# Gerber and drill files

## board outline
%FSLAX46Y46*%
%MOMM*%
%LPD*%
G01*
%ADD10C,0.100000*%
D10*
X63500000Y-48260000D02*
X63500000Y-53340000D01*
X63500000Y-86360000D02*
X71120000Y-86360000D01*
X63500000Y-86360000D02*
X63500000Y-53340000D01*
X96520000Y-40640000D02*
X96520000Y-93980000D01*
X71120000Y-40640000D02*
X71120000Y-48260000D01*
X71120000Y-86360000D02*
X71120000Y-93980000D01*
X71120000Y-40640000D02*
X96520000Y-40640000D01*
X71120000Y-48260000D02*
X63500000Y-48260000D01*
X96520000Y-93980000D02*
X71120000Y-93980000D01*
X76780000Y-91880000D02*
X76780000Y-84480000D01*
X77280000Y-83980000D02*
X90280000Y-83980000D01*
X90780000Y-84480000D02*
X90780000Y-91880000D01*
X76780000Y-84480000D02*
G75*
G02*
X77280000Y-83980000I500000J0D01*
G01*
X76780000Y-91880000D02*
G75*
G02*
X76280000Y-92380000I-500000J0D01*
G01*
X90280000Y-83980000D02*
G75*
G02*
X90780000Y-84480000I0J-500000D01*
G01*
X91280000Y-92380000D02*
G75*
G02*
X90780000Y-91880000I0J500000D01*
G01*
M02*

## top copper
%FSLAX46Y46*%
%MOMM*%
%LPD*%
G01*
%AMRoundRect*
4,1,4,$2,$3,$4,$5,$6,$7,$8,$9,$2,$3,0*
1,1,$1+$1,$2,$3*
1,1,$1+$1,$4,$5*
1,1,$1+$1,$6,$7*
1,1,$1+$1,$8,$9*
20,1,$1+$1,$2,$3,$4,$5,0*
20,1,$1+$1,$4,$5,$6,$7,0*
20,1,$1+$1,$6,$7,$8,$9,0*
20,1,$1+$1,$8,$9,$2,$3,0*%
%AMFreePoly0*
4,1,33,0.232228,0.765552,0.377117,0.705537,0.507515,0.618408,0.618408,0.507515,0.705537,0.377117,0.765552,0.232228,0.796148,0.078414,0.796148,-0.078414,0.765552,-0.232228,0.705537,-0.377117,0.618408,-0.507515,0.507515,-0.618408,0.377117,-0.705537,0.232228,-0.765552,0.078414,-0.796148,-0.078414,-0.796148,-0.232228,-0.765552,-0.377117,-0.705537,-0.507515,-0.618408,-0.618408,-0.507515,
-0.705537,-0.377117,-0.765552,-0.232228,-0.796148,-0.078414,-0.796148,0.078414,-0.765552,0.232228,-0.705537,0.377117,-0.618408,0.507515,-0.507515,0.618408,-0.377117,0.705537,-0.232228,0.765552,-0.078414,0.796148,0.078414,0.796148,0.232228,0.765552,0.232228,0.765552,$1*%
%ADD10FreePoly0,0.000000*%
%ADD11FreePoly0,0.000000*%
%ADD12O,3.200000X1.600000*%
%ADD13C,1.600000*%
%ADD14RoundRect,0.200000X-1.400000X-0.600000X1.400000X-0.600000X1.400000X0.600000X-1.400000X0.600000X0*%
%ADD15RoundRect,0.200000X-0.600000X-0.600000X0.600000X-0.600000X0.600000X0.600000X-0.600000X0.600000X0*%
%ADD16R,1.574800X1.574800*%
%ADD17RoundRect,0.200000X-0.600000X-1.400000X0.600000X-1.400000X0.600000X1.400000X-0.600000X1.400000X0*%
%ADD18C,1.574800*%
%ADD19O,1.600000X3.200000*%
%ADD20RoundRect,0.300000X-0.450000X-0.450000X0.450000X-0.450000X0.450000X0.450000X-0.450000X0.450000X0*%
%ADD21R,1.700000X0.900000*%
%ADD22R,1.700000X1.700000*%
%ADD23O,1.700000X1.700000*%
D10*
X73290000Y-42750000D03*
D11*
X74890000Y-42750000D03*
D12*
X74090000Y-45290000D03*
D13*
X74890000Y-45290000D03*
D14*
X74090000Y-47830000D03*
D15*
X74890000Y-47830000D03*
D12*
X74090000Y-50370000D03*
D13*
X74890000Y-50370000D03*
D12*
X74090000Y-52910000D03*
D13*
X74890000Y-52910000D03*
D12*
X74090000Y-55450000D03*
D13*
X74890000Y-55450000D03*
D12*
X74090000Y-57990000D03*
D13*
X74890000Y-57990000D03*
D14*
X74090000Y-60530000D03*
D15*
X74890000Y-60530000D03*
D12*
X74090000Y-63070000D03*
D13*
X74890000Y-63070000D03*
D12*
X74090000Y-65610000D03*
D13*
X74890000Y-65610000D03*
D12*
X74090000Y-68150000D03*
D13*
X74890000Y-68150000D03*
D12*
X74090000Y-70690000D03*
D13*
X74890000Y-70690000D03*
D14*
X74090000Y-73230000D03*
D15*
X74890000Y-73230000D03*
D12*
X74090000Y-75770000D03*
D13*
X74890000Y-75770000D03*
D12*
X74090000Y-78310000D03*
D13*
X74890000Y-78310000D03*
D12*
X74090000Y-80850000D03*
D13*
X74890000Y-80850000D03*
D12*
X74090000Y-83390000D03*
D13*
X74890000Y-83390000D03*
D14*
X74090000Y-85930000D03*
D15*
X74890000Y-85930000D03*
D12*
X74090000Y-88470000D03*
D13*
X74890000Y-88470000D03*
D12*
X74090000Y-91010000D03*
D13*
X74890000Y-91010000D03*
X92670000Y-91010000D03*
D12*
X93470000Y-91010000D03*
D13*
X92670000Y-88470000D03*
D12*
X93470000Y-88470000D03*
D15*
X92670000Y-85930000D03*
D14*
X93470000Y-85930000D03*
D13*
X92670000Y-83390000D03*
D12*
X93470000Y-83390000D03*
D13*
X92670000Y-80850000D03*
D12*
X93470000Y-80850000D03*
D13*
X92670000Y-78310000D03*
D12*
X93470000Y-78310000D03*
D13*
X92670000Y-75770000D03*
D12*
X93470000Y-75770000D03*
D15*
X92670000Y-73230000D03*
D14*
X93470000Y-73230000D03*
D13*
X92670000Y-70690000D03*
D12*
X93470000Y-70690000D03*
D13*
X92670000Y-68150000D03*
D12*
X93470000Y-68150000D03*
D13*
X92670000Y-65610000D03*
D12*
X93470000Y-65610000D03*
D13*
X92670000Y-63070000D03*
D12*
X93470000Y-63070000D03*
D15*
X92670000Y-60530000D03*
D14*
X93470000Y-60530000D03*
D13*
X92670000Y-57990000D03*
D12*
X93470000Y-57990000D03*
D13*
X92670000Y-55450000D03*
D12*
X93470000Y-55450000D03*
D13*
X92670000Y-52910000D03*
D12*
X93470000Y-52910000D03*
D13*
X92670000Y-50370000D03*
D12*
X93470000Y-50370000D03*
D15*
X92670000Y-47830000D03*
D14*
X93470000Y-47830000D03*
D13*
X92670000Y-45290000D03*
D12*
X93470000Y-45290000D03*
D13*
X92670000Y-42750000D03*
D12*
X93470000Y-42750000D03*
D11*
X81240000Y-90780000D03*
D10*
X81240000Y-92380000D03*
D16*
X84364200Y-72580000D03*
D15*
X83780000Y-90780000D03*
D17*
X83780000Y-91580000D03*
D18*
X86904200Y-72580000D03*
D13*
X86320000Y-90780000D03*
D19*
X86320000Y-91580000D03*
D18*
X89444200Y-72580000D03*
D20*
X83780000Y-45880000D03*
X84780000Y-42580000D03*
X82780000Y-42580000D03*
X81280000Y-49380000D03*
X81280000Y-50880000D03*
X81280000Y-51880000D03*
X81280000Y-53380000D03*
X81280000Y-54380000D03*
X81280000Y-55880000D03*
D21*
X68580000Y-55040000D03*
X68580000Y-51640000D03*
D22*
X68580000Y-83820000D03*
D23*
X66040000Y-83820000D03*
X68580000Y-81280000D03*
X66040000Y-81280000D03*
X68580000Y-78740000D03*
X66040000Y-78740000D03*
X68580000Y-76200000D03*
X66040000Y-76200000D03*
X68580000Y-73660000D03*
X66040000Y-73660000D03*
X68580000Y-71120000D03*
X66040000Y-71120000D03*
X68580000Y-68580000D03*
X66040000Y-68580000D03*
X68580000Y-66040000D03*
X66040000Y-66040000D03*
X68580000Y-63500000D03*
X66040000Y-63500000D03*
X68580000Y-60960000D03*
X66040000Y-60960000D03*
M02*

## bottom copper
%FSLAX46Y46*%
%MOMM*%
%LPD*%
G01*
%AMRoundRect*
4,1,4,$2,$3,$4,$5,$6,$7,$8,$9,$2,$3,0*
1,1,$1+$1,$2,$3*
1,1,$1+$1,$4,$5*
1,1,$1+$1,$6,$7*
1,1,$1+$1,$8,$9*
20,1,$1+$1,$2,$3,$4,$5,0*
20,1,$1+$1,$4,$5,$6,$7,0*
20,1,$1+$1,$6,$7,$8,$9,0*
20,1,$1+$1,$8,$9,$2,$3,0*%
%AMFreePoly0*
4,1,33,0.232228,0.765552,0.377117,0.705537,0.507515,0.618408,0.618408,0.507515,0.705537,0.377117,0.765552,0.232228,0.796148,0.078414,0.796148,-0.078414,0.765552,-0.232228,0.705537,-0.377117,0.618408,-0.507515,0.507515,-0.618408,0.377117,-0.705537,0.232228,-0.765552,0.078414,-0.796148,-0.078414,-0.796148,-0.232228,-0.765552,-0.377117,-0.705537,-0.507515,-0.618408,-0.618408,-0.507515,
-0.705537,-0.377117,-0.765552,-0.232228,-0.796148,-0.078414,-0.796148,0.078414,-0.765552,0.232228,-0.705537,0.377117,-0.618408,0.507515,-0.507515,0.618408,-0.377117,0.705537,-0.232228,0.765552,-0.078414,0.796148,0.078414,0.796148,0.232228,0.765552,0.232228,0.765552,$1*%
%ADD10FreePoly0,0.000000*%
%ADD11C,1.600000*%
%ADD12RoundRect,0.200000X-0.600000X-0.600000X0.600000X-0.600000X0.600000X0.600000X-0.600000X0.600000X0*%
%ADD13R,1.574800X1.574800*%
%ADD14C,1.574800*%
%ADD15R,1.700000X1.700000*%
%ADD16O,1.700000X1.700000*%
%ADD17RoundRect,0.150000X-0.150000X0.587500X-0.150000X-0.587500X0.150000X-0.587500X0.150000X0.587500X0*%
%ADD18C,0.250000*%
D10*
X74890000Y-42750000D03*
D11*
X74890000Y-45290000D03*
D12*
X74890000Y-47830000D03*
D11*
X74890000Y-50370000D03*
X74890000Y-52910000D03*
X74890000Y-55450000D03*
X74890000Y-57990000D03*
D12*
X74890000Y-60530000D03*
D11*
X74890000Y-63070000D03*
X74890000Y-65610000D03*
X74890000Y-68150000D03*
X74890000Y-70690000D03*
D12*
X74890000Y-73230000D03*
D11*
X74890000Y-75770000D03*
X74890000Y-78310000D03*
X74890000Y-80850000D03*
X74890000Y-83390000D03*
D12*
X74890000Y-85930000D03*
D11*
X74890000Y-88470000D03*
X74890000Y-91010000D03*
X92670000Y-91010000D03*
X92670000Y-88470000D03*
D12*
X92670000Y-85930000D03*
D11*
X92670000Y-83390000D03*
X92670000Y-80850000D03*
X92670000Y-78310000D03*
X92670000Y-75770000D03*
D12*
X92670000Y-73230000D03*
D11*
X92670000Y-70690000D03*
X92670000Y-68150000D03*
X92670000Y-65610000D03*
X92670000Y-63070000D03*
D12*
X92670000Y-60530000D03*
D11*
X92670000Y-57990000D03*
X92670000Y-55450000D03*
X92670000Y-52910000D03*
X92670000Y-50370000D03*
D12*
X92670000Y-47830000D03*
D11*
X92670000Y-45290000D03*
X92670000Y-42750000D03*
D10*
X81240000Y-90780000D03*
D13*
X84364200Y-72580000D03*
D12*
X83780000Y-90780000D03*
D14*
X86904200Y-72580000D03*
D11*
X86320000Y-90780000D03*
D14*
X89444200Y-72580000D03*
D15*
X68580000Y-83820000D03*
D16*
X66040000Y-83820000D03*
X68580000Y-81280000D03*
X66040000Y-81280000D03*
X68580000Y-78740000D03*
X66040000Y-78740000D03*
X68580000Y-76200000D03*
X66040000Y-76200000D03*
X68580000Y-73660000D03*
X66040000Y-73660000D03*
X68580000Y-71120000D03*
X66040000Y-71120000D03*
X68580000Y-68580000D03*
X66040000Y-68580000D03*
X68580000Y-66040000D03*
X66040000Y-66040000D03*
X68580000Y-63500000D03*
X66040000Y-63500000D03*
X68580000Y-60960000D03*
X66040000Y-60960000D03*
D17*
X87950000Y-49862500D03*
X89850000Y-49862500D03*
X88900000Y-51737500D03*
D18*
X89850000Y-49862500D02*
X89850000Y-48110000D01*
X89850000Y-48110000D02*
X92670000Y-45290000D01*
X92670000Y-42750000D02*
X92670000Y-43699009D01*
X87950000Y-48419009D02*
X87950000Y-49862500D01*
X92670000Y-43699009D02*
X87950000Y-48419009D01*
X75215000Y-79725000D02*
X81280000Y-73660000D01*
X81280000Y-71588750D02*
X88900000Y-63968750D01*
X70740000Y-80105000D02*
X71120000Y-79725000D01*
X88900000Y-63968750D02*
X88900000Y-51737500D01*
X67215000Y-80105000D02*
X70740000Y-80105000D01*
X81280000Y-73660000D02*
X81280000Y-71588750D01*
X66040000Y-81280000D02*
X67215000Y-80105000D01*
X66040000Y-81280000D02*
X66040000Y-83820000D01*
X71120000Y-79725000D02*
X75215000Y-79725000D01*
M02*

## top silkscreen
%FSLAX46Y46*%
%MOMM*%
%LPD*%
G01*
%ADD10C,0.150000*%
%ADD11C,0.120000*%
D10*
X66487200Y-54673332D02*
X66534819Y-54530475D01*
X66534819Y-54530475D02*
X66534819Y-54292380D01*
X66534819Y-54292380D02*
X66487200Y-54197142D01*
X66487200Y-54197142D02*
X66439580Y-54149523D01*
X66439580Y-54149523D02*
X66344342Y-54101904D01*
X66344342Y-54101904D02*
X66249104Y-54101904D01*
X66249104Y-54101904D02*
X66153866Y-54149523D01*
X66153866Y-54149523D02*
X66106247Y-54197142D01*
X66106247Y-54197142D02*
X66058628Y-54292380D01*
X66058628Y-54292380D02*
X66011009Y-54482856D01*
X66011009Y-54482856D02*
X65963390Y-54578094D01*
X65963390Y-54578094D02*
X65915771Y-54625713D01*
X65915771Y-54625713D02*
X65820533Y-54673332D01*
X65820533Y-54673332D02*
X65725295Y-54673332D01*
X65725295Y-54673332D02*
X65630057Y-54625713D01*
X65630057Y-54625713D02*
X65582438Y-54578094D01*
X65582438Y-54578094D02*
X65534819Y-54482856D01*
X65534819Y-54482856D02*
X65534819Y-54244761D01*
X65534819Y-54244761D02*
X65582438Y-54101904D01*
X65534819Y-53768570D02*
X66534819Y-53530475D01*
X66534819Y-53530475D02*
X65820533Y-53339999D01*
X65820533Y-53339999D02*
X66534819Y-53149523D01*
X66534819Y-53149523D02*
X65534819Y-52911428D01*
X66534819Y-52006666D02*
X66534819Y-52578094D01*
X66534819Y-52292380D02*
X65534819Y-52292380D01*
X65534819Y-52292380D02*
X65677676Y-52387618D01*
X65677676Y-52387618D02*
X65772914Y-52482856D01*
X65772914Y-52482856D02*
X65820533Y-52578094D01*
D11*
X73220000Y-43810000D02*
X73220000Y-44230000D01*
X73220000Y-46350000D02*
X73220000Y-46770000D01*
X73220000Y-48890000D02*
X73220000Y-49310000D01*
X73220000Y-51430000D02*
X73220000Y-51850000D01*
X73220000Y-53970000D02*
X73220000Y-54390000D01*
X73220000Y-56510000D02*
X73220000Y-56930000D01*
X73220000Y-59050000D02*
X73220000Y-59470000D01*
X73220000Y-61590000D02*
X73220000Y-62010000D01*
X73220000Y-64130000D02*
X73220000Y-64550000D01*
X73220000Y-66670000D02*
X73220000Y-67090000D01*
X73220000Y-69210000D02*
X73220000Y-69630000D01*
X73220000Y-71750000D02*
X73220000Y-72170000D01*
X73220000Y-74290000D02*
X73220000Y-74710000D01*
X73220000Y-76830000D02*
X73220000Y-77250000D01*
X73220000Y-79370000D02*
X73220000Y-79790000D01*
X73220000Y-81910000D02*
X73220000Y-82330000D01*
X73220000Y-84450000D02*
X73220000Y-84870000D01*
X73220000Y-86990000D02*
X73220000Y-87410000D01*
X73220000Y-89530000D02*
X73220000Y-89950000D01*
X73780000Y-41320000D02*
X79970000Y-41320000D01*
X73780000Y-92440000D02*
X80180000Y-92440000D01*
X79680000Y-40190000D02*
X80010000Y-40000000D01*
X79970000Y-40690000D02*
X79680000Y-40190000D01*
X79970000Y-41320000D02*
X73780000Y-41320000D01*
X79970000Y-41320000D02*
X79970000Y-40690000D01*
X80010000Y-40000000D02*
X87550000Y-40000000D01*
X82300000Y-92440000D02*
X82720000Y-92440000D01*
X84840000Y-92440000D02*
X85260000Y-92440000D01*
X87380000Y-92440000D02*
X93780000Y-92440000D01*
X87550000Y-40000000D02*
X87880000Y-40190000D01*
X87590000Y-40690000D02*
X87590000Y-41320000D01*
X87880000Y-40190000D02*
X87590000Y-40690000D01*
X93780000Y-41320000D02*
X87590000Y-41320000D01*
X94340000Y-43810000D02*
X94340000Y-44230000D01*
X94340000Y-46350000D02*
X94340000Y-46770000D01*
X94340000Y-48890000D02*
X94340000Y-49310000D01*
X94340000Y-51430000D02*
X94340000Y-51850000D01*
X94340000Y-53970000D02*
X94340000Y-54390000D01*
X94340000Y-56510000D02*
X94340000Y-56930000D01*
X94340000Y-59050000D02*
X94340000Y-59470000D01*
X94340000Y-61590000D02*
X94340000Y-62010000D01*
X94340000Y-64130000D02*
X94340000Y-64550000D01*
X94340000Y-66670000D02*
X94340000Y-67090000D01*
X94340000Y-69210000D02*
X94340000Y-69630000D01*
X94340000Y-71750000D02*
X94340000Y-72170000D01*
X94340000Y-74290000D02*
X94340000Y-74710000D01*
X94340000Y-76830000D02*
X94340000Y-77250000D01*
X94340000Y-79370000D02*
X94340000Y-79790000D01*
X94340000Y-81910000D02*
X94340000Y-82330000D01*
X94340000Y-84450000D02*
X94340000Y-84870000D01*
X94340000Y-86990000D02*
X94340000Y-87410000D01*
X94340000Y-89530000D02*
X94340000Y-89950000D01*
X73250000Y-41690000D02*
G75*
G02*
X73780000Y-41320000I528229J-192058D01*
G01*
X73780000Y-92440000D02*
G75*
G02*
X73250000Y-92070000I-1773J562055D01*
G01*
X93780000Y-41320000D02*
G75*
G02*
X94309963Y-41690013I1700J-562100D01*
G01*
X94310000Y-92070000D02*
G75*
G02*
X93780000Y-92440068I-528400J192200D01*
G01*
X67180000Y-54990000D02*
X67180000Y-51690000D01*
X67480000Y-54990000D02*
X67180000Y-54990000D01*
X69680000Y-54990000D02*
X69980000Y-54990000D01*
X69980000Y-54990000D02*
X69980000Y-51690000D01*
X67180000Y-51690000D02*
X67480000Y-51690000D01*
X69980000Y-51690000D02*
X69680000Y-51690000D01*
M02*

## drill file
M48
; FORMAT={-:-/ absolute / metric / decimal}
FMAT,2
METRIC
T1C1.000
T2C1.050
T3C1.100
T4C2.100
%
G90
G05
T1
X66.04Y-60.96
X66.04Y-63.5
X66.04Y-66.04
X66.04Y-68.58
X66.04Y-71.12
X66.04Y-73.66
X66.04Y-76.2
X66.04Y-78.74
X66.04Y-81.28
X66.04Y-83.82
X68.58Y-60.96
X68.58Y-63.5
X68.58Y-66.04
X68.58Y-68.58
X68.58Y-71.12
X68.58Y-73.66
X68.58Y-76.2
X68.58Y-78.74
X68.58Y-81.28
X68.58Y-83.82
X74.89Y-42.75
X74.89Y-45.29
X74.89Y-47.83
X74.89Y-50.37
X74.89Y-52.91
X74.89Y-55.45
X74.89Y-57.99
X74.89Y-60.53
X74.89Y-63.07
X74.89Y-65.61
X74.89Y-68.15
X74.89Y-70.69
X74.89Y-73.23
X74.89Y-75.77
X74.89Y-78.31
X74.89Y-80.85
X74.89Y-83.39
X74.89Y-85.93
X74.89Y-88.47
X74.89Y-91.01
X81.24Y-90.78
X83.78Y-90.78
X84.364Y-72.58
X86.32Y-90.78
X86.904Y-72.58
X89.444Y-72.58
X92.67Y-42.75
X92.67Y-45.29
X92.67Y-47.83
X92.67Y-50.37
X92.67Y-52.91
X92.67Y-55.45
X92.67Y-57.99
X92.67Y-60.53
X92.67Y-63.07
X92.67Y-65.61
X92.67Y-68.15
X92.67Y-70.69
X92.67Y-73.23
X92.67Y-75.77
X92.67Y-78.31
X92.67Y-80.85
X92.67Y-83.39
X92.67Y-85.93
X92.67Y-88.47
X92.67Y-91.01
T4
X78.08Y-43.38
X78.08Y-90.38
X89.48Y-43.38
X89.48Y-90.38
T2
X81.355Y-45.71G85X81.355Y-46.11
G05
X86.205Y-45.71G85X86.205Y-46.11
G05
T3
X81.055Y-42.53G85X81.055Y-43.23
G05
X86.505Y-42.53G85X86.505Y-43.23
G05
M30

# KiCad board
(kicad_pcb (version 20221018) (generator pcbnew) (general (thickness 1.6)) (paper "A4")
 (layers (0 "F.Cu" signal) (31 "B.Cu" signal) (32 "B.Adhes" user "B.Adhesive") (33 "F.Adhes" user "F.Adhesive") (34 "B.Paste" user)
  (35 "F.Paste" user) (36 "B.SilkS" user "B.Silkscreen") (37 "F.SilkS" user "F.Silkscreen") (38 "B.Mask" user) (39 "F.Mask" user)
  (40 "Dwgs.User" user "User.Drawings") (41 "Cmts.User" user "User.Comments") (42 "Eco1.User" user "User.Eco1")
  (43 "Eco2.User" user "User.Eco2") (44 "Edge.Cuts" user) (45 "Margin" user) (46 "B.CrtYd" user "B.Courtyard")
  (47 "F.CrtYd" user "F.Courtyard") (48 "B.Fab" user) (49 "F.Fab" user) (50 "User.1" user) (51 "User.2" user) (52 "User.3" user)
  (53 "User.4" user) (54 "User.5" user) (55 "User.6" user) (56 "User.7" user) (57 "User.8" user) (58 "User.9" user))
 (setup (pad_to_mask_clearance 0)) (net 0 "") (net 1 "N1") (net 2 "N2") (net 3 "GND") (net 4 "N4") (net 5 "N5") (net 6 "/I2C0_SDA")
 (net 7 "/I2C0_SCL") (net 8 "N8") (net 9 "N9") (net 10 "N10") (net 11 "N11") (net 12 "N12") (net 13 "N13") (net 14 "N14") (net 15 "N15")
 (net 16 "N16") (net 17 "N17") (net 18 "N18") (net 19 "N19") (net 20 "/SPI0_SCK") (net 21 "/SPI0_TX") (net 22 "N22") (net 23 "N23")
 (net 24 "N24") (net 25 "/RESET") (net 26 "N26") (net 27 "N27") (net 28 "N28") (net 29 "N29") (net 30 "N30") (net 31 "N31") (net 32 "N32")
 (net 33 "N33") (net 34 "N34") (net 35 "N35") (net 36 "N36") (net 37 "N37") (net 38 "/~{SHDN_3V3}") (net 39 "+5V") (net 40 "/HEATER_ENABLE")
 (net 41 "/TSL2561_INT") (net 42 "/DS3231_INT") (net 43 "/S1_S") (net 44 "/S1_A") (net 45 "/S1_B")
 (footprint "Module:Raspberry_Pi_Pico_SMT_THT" (layer "F.Cu") (at 74.89 42.75)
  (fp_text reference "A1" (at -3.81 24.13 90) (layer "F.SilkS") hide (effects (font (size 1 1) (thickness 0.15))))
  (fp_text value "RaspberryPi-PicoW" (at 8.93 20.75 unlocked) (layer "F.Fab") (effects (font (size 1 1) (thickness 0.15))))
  (fp_line (start -1.67 1.06) (end -1.67 1.48) (stroke (width 0.12) (type solid)) (layer "F.SilkS"))
  (fp_line (start -1.67 3.6) (end -1.67 4.02) (stroke (width 0.12) (type solid)) (layer "F.SilkS"))
  (fp_line (start -1.67 6.14) (end -1.67 6.56) (stroke (width 0.12) (type solid)) (layer "F.SilkS"))
  (fp_line (start -1.67 8.68) (end -1.67 9.1) (stroke (width 0.12) (type solid)) (layer "F.SilkS"))
  (fp_line (start -1.67 11.22) (end -1.67 11.64) (stroke (width 0.12) (type solid)) (layer "F.SilkS"))
  (fp_line (start -1.67 13.76) (end -1.67 14.18) (stroke (width 0.12) (type solid)) (layer "F.SilkS"))
  (fp_line (start -1.67 16.3) (end -1.67 16.72) (stroke (width 0.12) (type solid)) (layer "F.SilkS"))
  (fp_line (start -1.67 18.84) (end -1.67 19.26) (stroke (width 0.12) (type solid)) (layer "F.SilkS"))
  (fp_line (start -1.67 21.38) (end -1.67 21.8) (stroke (width 0.12) (type solid)) (layer "F.SilkS"))
  (fp_line (start -1.67 23.92) (end -1.67 24.34) (stroke (width 0.12) (type solid)) (layer "F.SilkS"))
  (fp_line (start -1.67 26.46) (end -1.67 26.88) (stroke (width 0.12) (type solid)) (layer "F.SilkS"))
  (fp_line (start -1.67 29) (end -1.67 29.42) (stroke (width 0.12) (type solid)) (layer "F.SilkS"))
  (fp_line (start -1.67 31.54) (end -1.67 31.96) (stroke (width 0.12) (type solid)) (layer "F.SilkS"))
  (fp_line (start -1.67 34.08) (end -1.67 34.5) (stroke (width 0.12) (type solid)) (layer "F.SilkS"))
  (fp_line (start -1.67 36.62) (end -1.67 37.04) (stroke (width 0.12) (type solid)) (layer "F.SilkS"))
  (fp_line (start -1.67 39.16) (end -1.67 39.58) (stroke (width 0.12) (type solid)) (layer "F.SilkS"))
  (fp_line (start -1.67 41.7) (end -1.67 42.12) (stroke (width 0.12) (type solid)) (layer "F.SilkS"))
  (fp_line (start -1.67 44.24) (end -1.67 44.66) (stroke (width 0.12) (type solid)) (layer "F.SilkS"))
  (fp_line (start -1.67 46.78) (end -1.67 47.2) (stroke (width 0.12) (type solid)) (layer "F.SilkS"))
  (fp_line (start -1.11 -1.43) (end 5.08 -1.43) (stroke (width 0.12) (type solid)) (layer "F.SilkS"))
  (fp_line (start -1.11 49.69) (end 5.29 49.69) (stroke (width 0.12) (type solid)) (layer "F.SilkS"))
  (fp_line (start 4.79 -2.56) (end 5.12 -2.75) (stroke (width 0.12) (type solid)) (layer "F.SilkS"))
  (fp_line (start 5.08 -2.06) (end 4.79 -2.56) (stroke (width 0.12) (type solid)) (layer "F.SilkS"))
  (fp_line (start 5.08 -1.43) (end -1.11 -1.43) (stroke (width 0.12) (type solid)) (layer "F.SilkS"))
  (fp_line (start 5.08 -1.43) (end 5.08 -2.06) (stroke (width 0.12) (type solid)) (layer "F.SilkS"))
  (fp_line (start 5.12 -2.75) (end 12.66 -2.75) (stroke (width 0.12) (type solid)) (layer "F.SilkS"))
  (fp_line (start 7.41 49.69) (end 7.83 49.69) (stroke (width 0.12) (type solid)) (layer "F.SilkS"))
  (fp_line (start 9.95 49.69) (end 10.37 49.69) (stroke (width 0.12) (type solid)) (layer "F.SilkS"))
  (fp_line (start 12.49 49.69) (end 18.89 49.69) (stroke (width 0.12) (type solid)) (layer "F.SilkS"))
  (fp_line (start 12.66 -2.75) (end 12.99 -2.56) (stroke (width 0.12) (type solid)) (layer "F.SilkS"))
  (fp_line (start 12.7 -2.06) (end 12.7 -1.43) (stroke (width 0.12) (type solid)) (layer "F.SilkS"))
  (fp_line (start 12.99 -2.56) (end 12.7 -2.06) (stroke (width 0.12) (type solid)) (layer "F.SilkS"))
  (fp_line (start 18.89 -1.43) (end 12.7 -1.43) (stroke (width 0.12) (type solid)) (layer "F.SilkS"))
  (fp_line (start 19.45 1.06) (end 19.45 1.48) (stroke (width 0.12) (type solid)) (layer "F.SilkS"))
  (fp_line (start 19.45 3.6) (end 19.45 4.02) (stroke (width 0.12) (type solid)) (layer "F.SilkS"))
  (fp_line (start 19.45 6.14) (end 19.45 6.56) (stroke (width 0.12) (type solid)) (layer "F.SilkS"))
  (fp_line (start 19.45 8.68) (end 19.45 9.1) (stroke (width 0.12) (type solid)) (layer "F.SilkS"))
  (fp_line (start 19.45 11.22) (end 19.45 11.64) (stroke (width 0.12) (type solid)) (layer "F.SilkS"))
  (fp_line (start 19.45 13.76) (end 19.45 14.18) (stroke (width 0.12) (type solid)) (layer "F.SilkS"))
  (fp_line (start 19.45 16.3) (end 19.45 16.72) (stroke (width 0.12) (type solid)) (layer "F.SilkS"))
  (fp_line (start 19.45 18.84) (end 19.45 19.26) (stroke (width 0.12) (type solid)) (layer "F.SilkS"))
  (fp_line (start 19.45 21.38) (end 19.45 21.8) (stroke (width 0.12) (type solid)) (layer "F.SilkS"))
  (fp_line (start 19.45 23.92) (end 19.45 24.34) (stroke (width 0.12) (type solid)) (layer "F.SilkS"))
  (fp_line (start 19.45 26.46) (end 19.45 26.88) (stroke (width 0.12) (type solid)) (layer "F.SilkS"))
  (fp_line (start 19.45 29) (end 19.45 29.42) (stroke (width 0.12) (type solid)) (layer "F.SilkS"))
  (fp_line (start 19.45 31.54) (end 19.45 31.96) (stroke (width 0.12) (type solid)) (layer "F.SilkS"))
  (fp_line (start 19.45 34.08) (end 19.45 34.5) (stroke (width 0.12) (type solid)) (layer "F.SilkS"))
  (fp_line (start 19.45 36.62) (end 19.45 37.04) (stroke (width 0.12) (type solid)) (layer "F.SilkS"))
  (fp_line (start 19.45 39.16) (end 19.45 39.58) (stroke (width 0.12) (type solid)) (layer "F.SilkS"))
  (fp_line (start 19.45 41.7) (end 19.45 42.12) (stroke (width 0.12) (type solid)) (layer "F.SilkS"))
  (fp_line (start 19.45 44.24) (end 19.45 44.66) (stroke (width 0.12) (type solid)) (layer "F.SilkS"))
  (fp_line (start 19.45 46.78) (end 19.45 47.2) (stroke (width 0.12) (type solid)) (layer "F.SilkS"))
  (fp_arc (start -1.64 -1.06) (mid -1.433508 -1.328808) (end -1.11 -1.43) (stroke (width 0.12) (type solid)) (layer "F.SilkS"))
  (fp_arc (start -1.11 49.69) (mid -1.433508 49.588809) (end -1.64 49.32) (stroke (width 0.12) (type solid)) (layer "F.SilkS"))
  (fp_arc (start 18.89 -1.43) (mid 19.213502 -1.328793) (end 19.42 -1.06) (stroke (width 0.12) (type solid)) (layer "F.SilkS"))
  (fp_arc (start 19.42 49.32) (mid 19.213487 49.588772) (end 18.89 49.69) (stroke (width 0.12) (type solid)) (layer "F.SilkS"))
  (fp_line (start 1.89 49.13) (end 1.89 41.73) (stroke (width 0.1) (type solid)) (layer "Edge.Cuts"))
  (fp_line (start 2.39 41.23) (end 15.39 41.23) (stroke (width 0.1) (type solid)) (layer "Edge.Cuts"))
  (fp_line (start 15.89 41.73) (end 15.89 49.13) (stroke (width 0.1) (type solid)) (layer "Edge.Cuts"))
  (fp_arc (start 1.89 41.73) (mid 2.036447 41.376447) (end 2.39 41.23) (stroke (width 0.1) (type solid)) (layer "Edge.Cuts"))
  (fp_arc (start 1.89 49.13) (mid 1.743553 49.483553) (end 1.39 49.63) (stroke (width 0.1) (type solid)) (layer "Edge.Cuts"))
  (fp_arc (start 15.39 41.23) (mid 15.743553 41.376447) (end 15.89 41.73) (stroke (width 0.1) (type solid)) (layer "Edge.Cuts"))
  (fp_arc (start 16.39 49.63) (mid 16.036447 49.483553) (end 15.89 49.13) (stroke (width 0.1) (type solid)) (layer "Edge.Cuts"))
  (pad "" np_thru_hole circle (at 3.19 0.63) (size 2.1 2.1) (drill 2.1) (layers "F&B.Cu" "*.Mask") (solder_mask_margin 0.85)
   (clearance 1.05))
  (pad "" np_thru_hole circle (at 3.19 47.63) (size 2.1 2.1) (drill 2.1) (layers "F&B.Cu" "*.Mask") (solder_mask_margin 0.85)
   (clearance 1.05))
  (pad "" np_thru_hole oval (at 6.165 0.13) (size 1.1 1.8) (drill oval 1.1 1.8) (layers "*.Mask"))
  (pad "" np_thru_hole oval (at 6.465 3.16) (size 1.05 1.45) (drill oval 1.05 1.45) (layers "*.Mask"))
  (pad "" np_thru_hole oval (at 11.315 3.16) (size 1.05 1.45) (drill oval 1.05 1.45) (layers "*.Mask"))
  (pad "" np_thru_hole oval (at 11.615 0.13) (size 1.1 1.8) (drill oval 1.1 1.8) (layers "*.Mask"))
  (pad "" np_thru_hole circle (at 14.59 0.63) (size 2.1 2.1) (drill 2.1) (layers "F&B.Cu" "*.Mask") (solder_mask_margin 0.85)
   (clearance 1.05))
  (pad "" np_thru_hole circle (at 14.59 47.63) (size 2.1 2.1) (drill 2.1) (layers "F&B.Cu" "*.Mask") (solder_mask_margin 0.85)
   (clearance 1.05))
  (pad "1" smd custom (at -1.6 0) (size 1.6 1.6) (layers "F.Cu" "F.Mask") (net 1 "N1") (thermal_bridge_angle 45)
   (options (clearance convexhull) (anchor circle)) (primitives))
  (pad "1" thru_hole custom (at 0 0) (size 1.6 1.6) (drill 1) (layers "*.Cu" "*.Mask") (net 1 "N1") (thermal_bridge_angle 45)
   (options (clearance convexhull) (anchor circle)) (primitives))
  (pad "2" smd oval (at -1.6 2.54) (size 3.2 1.6) (drill (offset 0.8 0)) (layers "F.Cu" "F.Mask") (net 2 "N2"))
  (pad "2" thru_hole circle (at 0 2.54) (size 1.6 1.6) (drill 1) (layers "*.Cu" "*.Mask") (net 2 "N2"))
  (pad "3" smd roundrect (at -1.6 5.08) (size 3.2 1.6) (drill (offset 0.8 0)) (layers "F.Cu" "F.Mask") (roundrect_rratio 0.125)
   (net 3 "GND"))
  (pad "3" thru_hole roundrect (at 0 5.08) (size 1.6 1.6) (drill 1) (layers "*.Cu" "*.Mask") (roundrect_rratio 0.125) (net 3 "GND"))
  (pad "4" smd oval (at -1.6 7.62) (size 3.2 1.6) (drill (offset 0.8 0)) (layers "F.Cu" "F.Mask") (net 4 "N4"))
  (pad "4" thru_hole circle (at 0 7.62) (size 1.6 1.6) (drill 1) (layers "*.Cu" "*.Mask") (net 4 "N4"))
  (pad "5" smd oval (at -1.6 10.16) (size 3.2 1.6) (drill (offset 0.8 0)) (layers "F.Cu" "F.Mask") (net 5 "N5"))
  (pad "5" thru_hole circle (at 0 10.16) (size 1.6 1.6) (drill 1) (layers "*.Cu" "*.Mask") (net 5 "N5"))
  (pad "6" smd oval (at -1.6 12.7) (size 3.2 1.6) (drill (offset 0.8 0)) (layers "F.Cu" "F.Mask") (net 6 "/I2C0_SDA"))
  (pad "6" thru_hole circle (at 0 12.7) (size 1.6 1.6) (drill 1) (layers "*.Cu" "*.Mask") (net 6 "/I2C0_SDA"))
  (pad "7" smd oval (at -1.6 15.24) (size 3.2 1.6) (drill (offset 0.8 0)) (layers "F.Cu" "F.Mask") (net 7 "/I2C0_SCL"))
  (pad "7" thru_hole circle (at 0 15.24) (size 1.6 1.6) (drill 1) (layers "*.Cu" "*.Mask") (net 7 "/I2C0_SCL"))
  (pad "8" smd roundrect (at -1.6 17.78) (size 3.2 1.6) (drill (offset 0.8 0)) (layers "F.Cu" "F.Mask") (roundrect_rratio 0.125)
   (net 3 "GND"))
  (pad "8" thru_hole roundrect (at 0 17.78) (size 1.6 1.6) (drill 1) (layers "*.Cu" "*.Mask") (roundrect_rratio 0.125) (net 3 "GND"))
  (pad "9" smd oval (at -1.6 20.32) (size 3.2 1.6) (drill (offset 0.8 0)) (layers "F.Cu" "F.Mask") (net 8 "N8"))
  (pad "9" thru_hole circle (at 0 20.32) (size 1.6 1.6) (drill 1) (layers "*.Cu" "*.Mask") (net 8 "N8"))
  (pad "10" smd oval (at -1.6 22.86) (size 3.2 1.6) (drill (offset 0.8 0)) (layers "F.Cu" "F.Mask") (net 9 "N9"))
  (pad "10" thru_hole circle (at 0 22.86) (size 1.6 1.6) (drill 1) (layers "*.Cu" "*.Mask") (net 9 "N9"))
  (pad "11" smd oval (at -1.6 25.4) (size 3.2 1.6) (drill (offset 0.8 0)) (layers "F.Cu" "F.Mask") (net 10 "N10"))
  (pad "11" thru_hole circle (at 0 25.4) (size 1.6 1.6) (drill 1) (layers "*.Cu" "*.Mask") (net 10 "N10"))
  (pad "12" smd oval (at -1.6 27.94) (size 3.2 1.6) (drill (offset 0.8 0)) (layers "F.Cu" "F.Mask") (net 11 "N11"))
  (pad "12" thru_hole circle (at 0 27.94) (size 1.6 1.6) (drill 1) (layers "*.Cu" "*.Mask") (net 11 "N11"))
  (pad "13" smd roundrect (at -1.6 30.48) (size 3.2 1.6) (drill (offset 0.8 0)) (layers "F.Cu" "F.Mask") (roundrect_rratio 0.125)
   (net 3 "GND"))
  (pad "13" thru_hole roundrect (at 0 30.48) (size 1.6 1.6) (drill 1) (layers "*.Cu" "*.Mask") (roundrect_rratio 0.125) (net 3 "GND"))
  (pad "14" smd oval (at -1.6 33.02) (size 3.2 1.6) (drill (offset 0.8 0)) (layers "F.Cu" "F.Mask") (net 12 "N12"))
  (pad "14" thru_hole circle (at 0 33.02) (size 1.6 1.6) (drill 1) (layers "*.Cu" "*.Mask") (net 12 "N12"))
  (pad "15" smd oval (at -1.6 35.56) (size 3.2 1.6) (drill (offset 0.8 0)) (layers "F.Cu" "F.Mask") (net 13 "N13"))
  (pad "15" thru_hole circle (at 0 35.56) (size 1.6 1.6) (drill 1) (layers "*.Cu" "*.Mask") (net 13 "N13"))
  (pad "16" smd oval (at -1.6 38.1) (size 3.2 1.6) (drill (offset 0.8 0)) (layers "F.Cu" "F.Mask") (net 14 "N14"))
  (pad "16" thru_hole circle (at 0 38.1) (size 1.6 1.6) (drill 1) (layers "*.Cu" "*.Mask") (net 14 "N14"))
  (pad "17" smd oval (at -1.6 40.64) (size 3.2 1.6) (drill (offset 0.8 0)) (layers "F.Cu" "F.Mask") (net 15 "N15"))
  (pad "17" thru_hole circle (at 0 40.64) (size 1.6 1.6) (drill 1) (layers "*.Cu" "*.Mask") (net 15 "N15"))
  (pad "18" smd roundrect (at -1.6 43.18) (size 3.2 1.6) (drill (offset 0.8 0)) (layers "F.Cu" "F.Mask") (roundrect_rratio 0.125)
   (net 3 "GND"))
  (pad "18" thru_hole roundrect (at 0 43.18) (size 1.6 1.6) (drill 1) (layers "*.Cu" "*.Mask") (roundrect_rratio 0.125) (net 3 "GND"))
  (pad "19" smd oval (at -1.6 45.72) (size 3.2 1.6) (drill (offset 0.8 0)) (layers "F.Cu" "F.Mask") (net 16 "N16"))
  (pad "19" thru_hole circle (at 0 45.72) (size 1.6 1.6) (drill 1) (layers "*.Cu" "*.Mask") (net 16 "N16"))
  (pad "20" smd oval (at -1.6 48.26) (size 3.2 1.6) (drill (offset 0.8 0)) (layers "F.Cu" "F.Mask") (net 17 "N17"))
  (pad "20" thru_hole circle (at 0 48.26) (size 1.6 1.6) (drill 1) (layers "*.Cu" "*.Mask") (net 17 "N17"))
  (pad "21" thru_hole circle (at 17.78 48.26) (size 1.6 1.6) (drill 1) (layers "*.Cu" "*.Mask") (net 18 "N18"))
  (pad "21" smd oval (at 19.38 48.26) (size 3.2 1.6) (drill (offset -0.8 0)) (layers "F.Cu" "F.Mask") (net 18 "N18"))
  (pad "22" thru_hole circle (at 17.78 45.72) (size 1.6 1.6) (drill 1) (layers "*.Cu" "*.Mask") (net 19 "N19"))
  (pad "22" smd oval (at 19.38 45.72) (size 3.2 1.6) (drill (offset -0.8 0)) (layers "F.Cu" "F.Mask") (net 19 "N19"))
  (pad "23" thru_hole roundrect (at 17.78 43.18) (size 1.6 1.6) (drill 1) (layers "*.Cu" "*.Mask") (roundrect_rratio 0.125) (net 3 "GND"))
  (pad "23" smd roundrect (at 19.38 43.18) (size 3.2 1.6) (drill (offset -0.8 0)) (layers "F.Cu" "F.Mask") (roundrect_rratio 0.125)
   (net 3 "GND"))
  (pad "24" thru_hole circle (at 17.78 40.64) (size 1.6 1.6) (drill 1) (layers "*.Cu" "*.Mask") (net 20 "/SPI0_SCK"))
  (pad "24" smd oval (at 19.38 40.64) (size 3.2 1.6) (drill (offset -0.8 0)) (layers "F.Cu" "F.Mask") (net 20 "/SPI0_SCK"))
  (pad "25" thru_hole circle (at 17.78 38.1) (size 1.6 1.6) (drill 1) (layers "*.Cu" "*.Mask") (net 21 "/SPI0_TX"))
  (pad "25" smd oval (at 19.38 38.1) (size 3.2 1.6) (drill (offset -0.8 0)) (layers "F.Cu" "F.Mask") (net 21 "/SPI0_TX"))
  (pad "26" thru_hole circle (at 17.78 35.56) (size 1.6 1.6) (drill 1) (layers "*.Cu" "*.Mask") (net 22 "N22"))
  (pad "26" smd oval (at 19.38 35.56) (size 3.2 1.6) (drill (offset -0.8 0)) (layers "F.Cu" "F.Mask") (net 22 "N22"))
  (pad "27" thru_hole circle (at 17.78 33.02) (size 1.6 1.6) (drill 1) (layers "*.Cu" "*.Mask") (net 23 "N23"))
  (pad "27" smd oval (at 19.38 33.02) (size 3.2 1.6) (drill (offset -0.8 0)) (layers "F.Cu" "F.Mask") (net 23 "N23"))
  (pad "28" thru_hole roundrect (at 17.78 30.48) (size 1.6 1.6) (drill 1) (layers "*.Cu" "*.Mask") (roundrect_rratio 0.125) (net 3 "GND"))
  (pad "28" smd roundrect (at 19.38 30.48) (size 3.2 1.6) (drill (offset -0.8 0)) (layers "F.Cu" "F.Mask") (roundrect_rratio 0.125)
   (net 3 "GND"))
  (pad "29" thru_hole circle (at 17.78 27.94) (size 1.6 1.6) (drill 1) (layers "*.Cu" "*.Mask") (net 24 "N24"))
  (pad "29" smd oval (at 19.38 27.94) (size 3.2 1.6) (drill (offset -0.8 0)) (layers "F.Cu" "F.Mask") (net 24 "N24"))
  (pad "30" thru_hole circle (at 17.78 25.4) (size 1.6 1.6) (drill 1) (layers "*.Cu" "*.Mask") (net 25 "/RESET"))
  (pad "30" smd oval (at 19.38 25.4) (size 3.2 1.6) (drill (offset -0.8 0)) (layers "F.Cu" "F.Mask") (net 25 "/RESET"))
  (pad "31" thru_hole circle (at 17.78 22.86) (size 1.6 1.6) (drill 1) (layers "*.Cu" "*.Mask") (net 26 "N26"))
  (pad "31" smd oval (at 19.38 22.86) (size 3.2 1.6) (drill (offset -0.8 0)) (layers "F.Cu" "F.Mask") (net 26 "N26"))
  (pad "32" thru_hole circle (at 17.78 20.32) (size 1.6 1.6) (drill 1) (layers "*.Cu" "*.Mask") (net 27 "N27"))
  (pad "32" smd oval (at 19.38 20.32) (size 3.2 1.6) (drill (offset -0.8 0)) (layers "F.Cu" "F.Mask") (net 27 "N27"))
  (pad "33" thru_hole roundrect (at 17.78 17.78) (size 1.6 1.6) (drill 1) (layers "*.Cu" "*.Mask") (roundrect_rratio 0.125) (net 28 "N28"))
  (pad "33" smd roundrect (at 19.38 17.78) (size 3.2 1.6) (drill (offset -0.8 0)) (layers "F.Cu" "F.Mask") (roundrect_rratio 0.125)
   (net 28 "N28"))
  (pad "34" thru_hole circle (at 17.78 15.24) (size 1.6 1.6) (drill 1) (layers "*.Cu" "*.Mask") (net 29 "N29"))
  (pad "34" smd oval (at 19.38 15.24) (size 3.2 1.6) (drill (offset -0.8 0)) (layers "F.Cu" "F.Mask") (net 29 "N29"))
  (pad "35" thru_hole circle (at 17.78 12.7) (size 1.6 1.6) (drill 1) (layers "*.Cu" "*.Mask") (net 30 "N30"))
  (pad "35" smd oval (at 19.38 12.7) (size 3.2 1.6) (drill (offset -0.8 0)) (layers "F.Cu" "F.Mask") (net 30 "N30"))
  (pad "36" thru_hole circle (at 17.78 10.16) (size 1.6 1.6) (drill 1) (layers "*.Cu" "*.Mask") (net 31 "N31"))
  (pad "36" smd oval (at 19.38 10.16) (size 3.2 1.6) (drill (offset -0.8 0)) (layers "F.Cu" "F.Mask") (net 31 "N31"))
  (pad "37" thru_hole circle (at 17.78 7.62) (size 1.6 1.6) (drill 1) (layers "*.Cu" "*.Mask") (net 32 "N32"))
  (pad "37" smd oval (at 19.38 7.62) (size 3.2 1.6) (drill (offset -0.8 0)) (layers "F.Cu" "F.Mask") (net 32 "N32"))
  (pad "38" thru_hole roundrect (at 17.78 5.08) (size 1.6 1.6) (drill 1) (layers "*.Cu" "*.Mask") (roundrect_rratio 0.125) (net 3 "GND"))
  (pad "38" smd roundrect (at 19.38 5.08) (size 3.2 1.6) (drill (offset -0.8 0)) (layers "F.Cu" "F.Mask") (roundrect_rratio 0.125)
   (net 3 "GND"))
  (pad "39" thru_hole circle (at 17.78 2.54) (size 1.6 1.6) (drill 1) (layers "*.Cu" "*.Mask") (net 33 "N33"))
  (pad "39" smd oval (at 19.38 2.54) (size 3.2 1.6) (drill (offset -0.8 0)) (layers "F.Cu" "F.Mask") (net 33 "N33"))
  (pad "40" thru_hole circle (at 17.78 0) (size 1.6 1.6) (drill 1) (layers "*.Cu" "*.Mask") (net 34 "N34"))
  (pad "40" smd oval (at 19.38 0) (size 3.2 1.6) (drill (offset -0.8 0)) (layers "F.Cu" "F.Mask") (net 34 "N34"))
  (pad "41" thru_hole custom (at 6.35 48.03) (size 1.6 1.6) (drill 1) (layers "*.Cu" "*.Mask") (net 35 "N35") (thermal_bridge_angle 45)
   (options (clearance convexhull) (anchor circle)) (primitives))
  (pad "41" smd custom (at 6.35 49.63) (size 1.6 1.6) (layers "F.Cu" "F.Mask") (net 35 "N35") (thermal_bridge_angle 45)
   (options (clearance convexhull) (anchor circle)) (primitives))
  (pad "41" thru_hole rect (at 9.4742 29.83) (size 1.5748 1.5748) (drill 1) (layers "*.Cu" "*.Mask") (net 35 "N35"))
  (pad "42" thru_hole roundrect (at 8.89 48.03) (size 1.6 1.6) (drill 1) (layers "*.Cu" "*.Mask") (roundrect_rratio 0.125) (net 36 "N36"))
  (pad "42" smd roundrect (at 8.89 49.63) (size 1.6 3.2) (drill (offset 0 -0.8)) (layers "F.Cu" "F.Mask") (roundrect_rratio 0.125)
   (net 36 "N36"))
  (pad "42" thru_hole circle (at 12.0142 29.83) (size 1.5748 1.5748) (drill 1) (layers "*.Cu" "*.Mask") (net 36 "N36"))
  (pad "43" thru_hole circle (at 11.43 48.03) (size 1.6 1.6) (drill 1) (layers "*.Cu" "*.Mask") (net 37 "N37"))
  (pad "43" smd oval (at 11.43 49.63) (size 1.6 3.2) (drill (offset 0 -0.8)) (layers "F.Cu" "F.Mask") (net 37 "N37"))
  (pad "43" thru_hole circle (at 14.5542 29.83) (size 1.5748 1.5748) (drill 1) (layers "*.Cu" "*.Mask") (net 37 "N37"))
  (pad "51" smd roundrect (at 8.89 3.13) (size 1.5 1.5) (layers "F.Cu" "F.Mask") (roundrect_rratio 0.2))
  (pad "52" smd roundrect (at 9.89 -0.17) (size 1.5 1.5) (layers "F.Cu" "F.Mask") (roundrect_rratio 0.2))
  (pad "53" smd roundrect (at 7.89 -0.17) (size 1.5 1.5) (layers "F.Cu" "F.Mask") (roundrect_rratio 0.2))
  (pad "54" smd roundrect (at 6.39 6.63) (size 1.5 1.5) (layers "F.Cu" "F.Mask") (roundrect_rratio 0.2))
  (pad "54" smd roundrect (at 6.39 8.13) (size 1.5 1.5) (layers "F.Cu" "F.Mask") (roundrect_rratio 0.2))
  (pad "55" smd roundrect (at 6.39 9.13) (size 1.5 1.5) (layers "F.Cu" "F.Mask") (roundrect_rratio 0.2))
  (pad "55" smd roundrect (at 6.39 10.63) (size 1.5 1.5) (layers "F.Cu" "F.Mask") (roundrect_rratio 0.2))
  (pad "56" smd roundrect (at 6.39 11.63) (size 1.5 1.5) (layers "F.Cu" "F.Mask") (roundrect_rratio 0.2))
  (pad "56" smd roundrect (at 6.39 13.13) (size 1.5 1.5) (layers "F.Cu" "F.Mask") (roundrect_rratio 0.2))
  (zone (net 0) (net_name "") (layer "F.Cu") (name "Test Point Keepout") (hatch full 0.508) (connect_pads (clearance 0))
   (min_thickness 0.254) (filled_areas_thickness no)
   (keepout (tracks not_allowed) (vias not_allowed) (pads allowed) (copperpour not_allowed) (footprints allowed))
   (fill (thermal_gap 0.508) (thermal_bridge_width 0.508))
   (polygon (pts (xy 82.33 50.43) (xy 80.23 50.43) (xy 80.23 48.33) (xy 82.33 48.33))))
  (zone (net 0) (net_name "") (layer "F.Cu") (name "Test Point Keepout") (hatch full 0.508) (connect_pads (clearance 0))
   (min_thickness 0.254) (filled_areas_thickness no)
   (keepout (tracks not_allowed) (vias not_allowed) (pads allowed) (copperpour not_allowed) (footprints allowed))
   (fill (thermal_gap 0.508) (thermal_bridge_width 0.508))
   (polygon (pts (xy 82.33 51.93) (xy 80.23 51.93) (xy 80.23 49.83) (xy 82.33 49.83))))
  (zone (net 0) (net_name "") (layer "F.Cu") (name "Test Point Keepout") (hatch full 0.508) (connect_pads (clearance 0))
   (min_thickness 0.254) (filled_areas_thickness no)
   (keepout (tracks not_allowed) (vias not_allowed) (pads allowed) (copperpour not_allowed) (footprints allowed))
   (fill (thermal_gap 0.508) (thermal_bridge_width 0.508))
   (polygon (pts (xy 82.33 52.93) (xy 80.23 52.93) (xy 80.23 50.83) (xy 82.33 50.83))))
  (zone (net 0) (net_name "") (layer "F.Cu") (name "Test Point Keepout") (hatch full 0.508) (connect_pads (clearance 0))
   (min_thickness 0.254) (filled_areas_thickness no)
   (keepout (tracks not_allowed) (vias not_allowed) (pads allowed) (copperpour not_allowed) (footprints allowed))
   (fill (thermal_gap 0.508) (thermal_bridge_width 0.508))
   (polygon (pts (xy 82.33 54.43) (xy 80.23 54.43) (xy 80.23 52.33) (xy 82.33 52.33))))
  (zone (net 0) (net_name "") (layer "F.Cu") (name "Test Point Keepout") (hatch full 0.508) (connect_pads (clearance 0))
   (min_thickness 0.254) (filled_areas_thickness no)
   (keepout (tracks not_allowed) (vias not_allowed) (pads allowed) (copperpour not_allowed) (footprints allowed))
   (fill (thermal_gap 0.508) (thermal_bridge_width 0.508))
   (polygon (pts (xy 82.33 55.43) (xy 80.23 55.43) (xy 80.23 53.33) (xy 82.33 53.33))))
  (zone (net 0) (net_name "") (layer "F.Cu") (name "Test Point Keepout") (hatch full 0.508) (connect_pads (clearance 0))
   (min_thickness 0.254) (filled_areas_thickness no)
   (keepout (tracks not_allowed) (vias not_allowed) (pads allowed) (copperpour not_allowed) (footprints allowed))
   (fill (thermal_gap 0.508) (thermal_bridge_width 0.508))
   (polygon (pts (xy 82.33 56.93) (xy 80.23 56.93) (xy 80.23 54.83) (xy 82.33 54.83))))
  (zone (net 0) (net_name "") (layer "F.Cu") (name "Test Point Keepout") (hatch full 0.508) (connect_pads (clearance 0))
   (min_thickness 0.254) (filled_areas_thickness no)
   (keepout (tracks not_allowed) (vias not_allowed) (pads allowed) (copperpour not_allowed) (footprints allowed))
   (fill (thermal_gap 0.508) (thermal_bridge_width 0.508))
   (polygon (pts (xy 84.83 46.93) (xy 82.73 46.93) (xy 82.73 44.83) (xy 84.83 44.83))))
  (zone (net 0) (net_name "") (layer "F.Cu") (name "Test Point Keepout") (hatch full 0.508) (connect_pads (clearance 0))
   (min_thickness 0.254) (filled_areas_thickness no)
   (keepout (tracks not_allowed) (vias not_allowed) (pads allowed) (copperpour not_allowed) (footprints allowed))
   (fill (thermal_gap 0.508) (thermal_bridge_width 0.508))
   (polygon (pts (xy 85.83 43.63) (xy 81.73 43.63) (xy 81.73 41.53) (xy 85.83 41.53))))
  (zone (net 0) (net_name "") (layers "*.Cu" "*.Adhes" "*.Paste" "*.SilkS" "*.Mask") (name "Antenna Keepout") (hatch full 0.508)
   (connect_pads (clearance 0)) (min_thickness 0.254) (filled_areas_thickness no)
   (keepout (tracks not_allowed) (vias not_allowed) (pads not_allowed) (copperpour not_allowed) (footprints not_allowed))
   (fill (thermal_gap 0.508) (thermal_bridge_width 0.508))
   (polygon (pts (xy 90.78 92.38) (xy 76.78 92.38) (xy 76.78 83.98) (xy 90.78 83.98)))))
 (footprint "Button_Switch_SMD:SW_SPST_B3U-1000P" (layer "F.Cu") (at 68.58 53.34 90)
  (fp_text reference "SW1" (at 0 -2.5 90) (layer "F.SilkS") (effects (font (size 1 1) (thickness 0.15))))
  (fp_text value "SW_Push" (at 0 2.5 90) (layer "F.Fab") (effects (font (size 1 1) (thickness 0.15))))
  (fp_line (start -1.65 -1.4) (end 1.65 -1.4) (stroke (width 0.12) (type solid)) (layer "F.SilkS"))
  (fp_line (start -1.65 -1.1) (end -1.65 -1.4) (stroke (width 0.12) (type solid)) (layer "F.SilkS"))
  (fp_line (start -1.65 1.1) (end -1.65 1.4) (stroke (width 0.12) (type solid)) (layer "F.SilkS"))
  (fp_line (start -1.65 1.4) (end 1.65 1.4) (stroke (width 0.12) (type solid)) (layer "F.SilkS"))
  (fp_line (start 1.65 -1.4) (end 1.65 -1.1) (stroke (width 0.12) (type solid)) (layer "F.SilkS"))
  (fp_line (start 1.65 1.4) (end 1.65 1.1) (stroke (width 0.12) (type solid)) (layer "F.SilkS"))
  (pad "1" smd rect (at -1.7 0 90) (size 0.9 1.7) (layers "F.Cu" "F.Paste" "F.Mask") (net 25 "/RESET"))
  (pad "2" smd rect (at 1.7 0 90) (size 0.9 1.7) (layers "F.Cu" "F.Paste" "F.Mask") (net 3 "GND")))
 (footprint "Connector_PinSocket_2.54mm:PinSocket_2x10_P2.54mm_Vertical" (layer "B.Cu") (at 68.58 83.82)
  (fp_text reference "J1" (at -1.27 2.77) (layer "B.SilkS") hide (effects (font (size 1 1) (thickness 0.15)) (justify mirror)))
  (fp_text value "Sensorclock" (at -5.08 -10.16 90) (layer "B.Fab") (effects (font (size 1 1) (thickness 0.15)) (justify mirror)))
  (pad "1" thru_hole rect (at 0 0) (size 1.7 1.7) (drill 1) (layers "*.Cu" "*.Mask") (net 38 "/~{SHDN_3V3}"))
  (pad "2" thru_hole oval (at -2.54 0) (size 1.7 1.7) (drill 1) (layers "*.Cu" "*.Mask") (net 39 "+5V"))
  (pad "3" thru_hole oval (at 0 -2.54) (size 1.7 1.7) (drill 1) (layers "*.Cu" "*.Mask") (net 6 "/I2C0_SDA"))
  (pad "4" thru_hole oval (at -2.54 -2.54) (size 1.7 1.7) (drill 1) (layers "*.Cu" "*.Mask") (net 39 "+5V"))
  (pad "5" thru_hole oval (at 0 -5.08) (size 1.7 1.7) (drill 1) (layers "*.Cu" "*.Mask") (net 7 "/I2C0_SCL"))
  (pad "6" thru_hole oval (at -2.54 -5.08) (size 1.7 1.7) (drill 1) (layers "*.Cu" "*.Mask") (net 3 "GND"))
  (pad "7" thru_hole oval (at 0 -7.62) (size 1.7 1.7) (drill 1) (layers "*.Cu" "*.Mask") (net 21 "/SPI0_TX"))
  (pad "8" thru_hole oval (at -2.54 -7.62) (size 1.7 1.7) (drill 1) (layers "*.Cu" "*.Mask") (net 3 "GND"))
  (pad "9" thru_hole oval (at 0 -10.16) (size 1.7 1.7) (drill 1) (layers "*.Cu" "*.Mask") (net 20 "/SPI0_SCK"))
  (pad "10" thru_hole oval (at -2.54 -10.16) (size 1.7 1.7) (drill 1) (layers "*.Cu" "*.Mask") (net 3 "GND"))
  (pad "11" thru_hole oval (at 0 -12.7) (size 1.7 1.7) (drill 1) (layers "*.Cu" "*.Mask") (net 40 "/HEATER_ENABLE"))
  (pad "12" thru_hole oval (at -2.54 -12.7) (size 1.7 1.7) (drill 1) (layers "*.Cu" "*.Mask") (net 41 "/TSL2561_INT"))
  (pad "13" thru_hole oval (at 0 -15.24) (size 1.7 1.7) (drill 1) (layers "*.Cu" "*.Mask") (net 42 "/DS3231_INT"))
  (pad "14" thru_hole oval (at -2.54 -15.24) (size 1.7 1.7) (drill 1) (layers "*.Cu" "*.Mask") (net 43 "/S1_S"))
  (pad "15" thru_hole oval (at 0 -17.78) (size 1.7 1.7) (drill 1) (layers "*.Cu" "*.Mask") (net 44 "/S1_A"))
  (pad "16" thru_hole oval (at -2.54 -17.78) (size 1.7 1.7) (drill 1) (layers "*.Cu" "*.Mask") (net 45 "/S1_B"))
  (pad "17" thru_hole oval (at 0 -20.32) (size 1.7 1.7) (drill 1) (layers "*.Cu" "*.Mask") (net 3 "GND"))
  (pad "18" thru_hole oval (at -2.54 -20.32) (size 1.7 1.7) (drill 1) (layers "*.Cu" "*.Mask") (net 3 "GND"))
  (pad "19" thru_hole oval (at 0 -22.86) (size 1.7 1.7) (drill 1) (layers "*.Cu" "*.Mask") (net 3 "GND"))
  (pad "20" thru_hole oval (at -2.54 -22.86) (size 1.7 1.7) (drill 1) (layers "*.Cu" "*.Mask") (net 3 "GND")))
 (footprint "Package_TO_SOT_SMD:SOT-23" (layer "B.Cu") (at 88.9 50.8 -90)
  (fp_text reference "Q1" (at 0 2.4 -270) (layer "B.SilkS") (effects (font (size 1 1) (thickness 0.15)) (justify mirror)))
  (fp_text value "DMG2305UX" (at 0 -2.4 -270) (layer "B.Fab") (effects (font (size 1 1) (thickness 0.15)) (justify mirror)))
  (pad "1" smd roundrect (at -0.9375 0.95 270) (size 1.475 0.6) (layers "B.Cu" "B.Paste" "B.Mask") (roundrect_rratio 0.25) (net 34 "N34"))
  (pad "2" smd roundrect (at -0.9375 -0.95 270) (size 1.475 0.6) (layers "B.Cu" "B.Paste" "B.Mask") (roundrect_rratio 0.25) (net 33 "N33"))
  (pad "3" smd roundrect (at 0.9375 0 270) (size 1.475 0.6) (layers "B.Cu" "B.Paste" "B.Mask") (roundrect_rratio 0.25) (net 39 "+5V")))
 (gr_line (start 63.5 48.26) (end 63.5 53.34) (stroke (width 0.1) (type default)) (layer "Edge.Cuts"))
 (gr_line (start 63.5 86.36) (end 71.12 86.36) (stroke (width 0.1) (type default)) (layer "Edge.Cuts"))
 (gr_line (start 63.5 86.36) (end 63.5 53.34) (stroke (width 0.1) (type default)) (layer "Edge.Cuts"))
 (gr_line (start 96.52 40.64) (end 96.52 93.98) (stroke (width 0.1) (type default)) (layer "Edge.Cuts"))
 (gr_line (start 71.12 40.64) (end 71.12 48.26) (stroke (width 0.1) (type default)) (layer "Edge.Cuts"))
 (gr_line (start 71.12 86.36) (end 71.12 93.98) (stroke (width 0.1) (type default)) (layer "Edge.Cuts"))
 (gr_line (start 71.12 40.64) (end 96.52 40.64) (stroke (width 0.1) (type default)) (layer "Edge.Cuts"))
 (gr_line (start 71.12 48.26) (end 63.5 48.26) (stroke (width 0.1) (type default)) (layer "Edge.Cuts"))
 (gr_line (start 96.52 93.98) (end 71.12 93.98) (stroke (width 0.1) (type default)) (layer "Edge.Cuts"))
 (segment (start 89.85 49.8625) (end 89.85 48.11) (width 0.25) (layer "B.Cu") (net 33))
 (segment (start 89.85 48.11) (end 92.67 45.29) (width 0.25) (layer "B.Cu") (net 33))
 (segment (start 92.67 42.75) (end 92.67 43.699009) (width 0.25) (layer "B.Cu") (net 34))
 (segment (start 87.95 48.419009) (end 87.95 49.8625) (width 0.25) (layer "B.Cu") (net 34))
 (segment (start 92.67 43.699009) (end 87.95 48.419009) (width 0.25) (layer "B.Cu") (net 34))
 (segment (start 75.215 79.725) (end 81.28 73.66) (width 0.25) (layer "B.Cu") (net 39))
 (segment (start 81.28 71.58875) (end 88.9 63.96875) (width 0.25) (layer "B.Cu") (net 39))
 (segment (start 70.74 80.105) (end 71.12 79.725) (width 0.25) (layer "B.Cu") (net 39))
 (segment (start 88.9 63.96875) (end 88.9 51.7375) (width 0.25) (layer "B.Cu") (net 39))
 (segment (start 67.215 80.105) (end 70.74 80.105) (width 0.25) (layer "B.Cu") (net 39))
 (segment (start 81.28 73.66) (end 81.28 71.58875) (width 0.25) (layer "B.Cu") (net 39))
 (segment (start 66.04 81.28) (end 67.215 80.105) (width 0.25) (layer "B.Cu") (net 39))
 (segment (start 66.04 81.28) (end 66.04 83.82) (width 0.25) (layer "B.Cu") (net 39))
 (segment (start 71.12 79.725) (end 75.215 79.725) (width 0.25) (layer "B.Cu") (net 39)))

